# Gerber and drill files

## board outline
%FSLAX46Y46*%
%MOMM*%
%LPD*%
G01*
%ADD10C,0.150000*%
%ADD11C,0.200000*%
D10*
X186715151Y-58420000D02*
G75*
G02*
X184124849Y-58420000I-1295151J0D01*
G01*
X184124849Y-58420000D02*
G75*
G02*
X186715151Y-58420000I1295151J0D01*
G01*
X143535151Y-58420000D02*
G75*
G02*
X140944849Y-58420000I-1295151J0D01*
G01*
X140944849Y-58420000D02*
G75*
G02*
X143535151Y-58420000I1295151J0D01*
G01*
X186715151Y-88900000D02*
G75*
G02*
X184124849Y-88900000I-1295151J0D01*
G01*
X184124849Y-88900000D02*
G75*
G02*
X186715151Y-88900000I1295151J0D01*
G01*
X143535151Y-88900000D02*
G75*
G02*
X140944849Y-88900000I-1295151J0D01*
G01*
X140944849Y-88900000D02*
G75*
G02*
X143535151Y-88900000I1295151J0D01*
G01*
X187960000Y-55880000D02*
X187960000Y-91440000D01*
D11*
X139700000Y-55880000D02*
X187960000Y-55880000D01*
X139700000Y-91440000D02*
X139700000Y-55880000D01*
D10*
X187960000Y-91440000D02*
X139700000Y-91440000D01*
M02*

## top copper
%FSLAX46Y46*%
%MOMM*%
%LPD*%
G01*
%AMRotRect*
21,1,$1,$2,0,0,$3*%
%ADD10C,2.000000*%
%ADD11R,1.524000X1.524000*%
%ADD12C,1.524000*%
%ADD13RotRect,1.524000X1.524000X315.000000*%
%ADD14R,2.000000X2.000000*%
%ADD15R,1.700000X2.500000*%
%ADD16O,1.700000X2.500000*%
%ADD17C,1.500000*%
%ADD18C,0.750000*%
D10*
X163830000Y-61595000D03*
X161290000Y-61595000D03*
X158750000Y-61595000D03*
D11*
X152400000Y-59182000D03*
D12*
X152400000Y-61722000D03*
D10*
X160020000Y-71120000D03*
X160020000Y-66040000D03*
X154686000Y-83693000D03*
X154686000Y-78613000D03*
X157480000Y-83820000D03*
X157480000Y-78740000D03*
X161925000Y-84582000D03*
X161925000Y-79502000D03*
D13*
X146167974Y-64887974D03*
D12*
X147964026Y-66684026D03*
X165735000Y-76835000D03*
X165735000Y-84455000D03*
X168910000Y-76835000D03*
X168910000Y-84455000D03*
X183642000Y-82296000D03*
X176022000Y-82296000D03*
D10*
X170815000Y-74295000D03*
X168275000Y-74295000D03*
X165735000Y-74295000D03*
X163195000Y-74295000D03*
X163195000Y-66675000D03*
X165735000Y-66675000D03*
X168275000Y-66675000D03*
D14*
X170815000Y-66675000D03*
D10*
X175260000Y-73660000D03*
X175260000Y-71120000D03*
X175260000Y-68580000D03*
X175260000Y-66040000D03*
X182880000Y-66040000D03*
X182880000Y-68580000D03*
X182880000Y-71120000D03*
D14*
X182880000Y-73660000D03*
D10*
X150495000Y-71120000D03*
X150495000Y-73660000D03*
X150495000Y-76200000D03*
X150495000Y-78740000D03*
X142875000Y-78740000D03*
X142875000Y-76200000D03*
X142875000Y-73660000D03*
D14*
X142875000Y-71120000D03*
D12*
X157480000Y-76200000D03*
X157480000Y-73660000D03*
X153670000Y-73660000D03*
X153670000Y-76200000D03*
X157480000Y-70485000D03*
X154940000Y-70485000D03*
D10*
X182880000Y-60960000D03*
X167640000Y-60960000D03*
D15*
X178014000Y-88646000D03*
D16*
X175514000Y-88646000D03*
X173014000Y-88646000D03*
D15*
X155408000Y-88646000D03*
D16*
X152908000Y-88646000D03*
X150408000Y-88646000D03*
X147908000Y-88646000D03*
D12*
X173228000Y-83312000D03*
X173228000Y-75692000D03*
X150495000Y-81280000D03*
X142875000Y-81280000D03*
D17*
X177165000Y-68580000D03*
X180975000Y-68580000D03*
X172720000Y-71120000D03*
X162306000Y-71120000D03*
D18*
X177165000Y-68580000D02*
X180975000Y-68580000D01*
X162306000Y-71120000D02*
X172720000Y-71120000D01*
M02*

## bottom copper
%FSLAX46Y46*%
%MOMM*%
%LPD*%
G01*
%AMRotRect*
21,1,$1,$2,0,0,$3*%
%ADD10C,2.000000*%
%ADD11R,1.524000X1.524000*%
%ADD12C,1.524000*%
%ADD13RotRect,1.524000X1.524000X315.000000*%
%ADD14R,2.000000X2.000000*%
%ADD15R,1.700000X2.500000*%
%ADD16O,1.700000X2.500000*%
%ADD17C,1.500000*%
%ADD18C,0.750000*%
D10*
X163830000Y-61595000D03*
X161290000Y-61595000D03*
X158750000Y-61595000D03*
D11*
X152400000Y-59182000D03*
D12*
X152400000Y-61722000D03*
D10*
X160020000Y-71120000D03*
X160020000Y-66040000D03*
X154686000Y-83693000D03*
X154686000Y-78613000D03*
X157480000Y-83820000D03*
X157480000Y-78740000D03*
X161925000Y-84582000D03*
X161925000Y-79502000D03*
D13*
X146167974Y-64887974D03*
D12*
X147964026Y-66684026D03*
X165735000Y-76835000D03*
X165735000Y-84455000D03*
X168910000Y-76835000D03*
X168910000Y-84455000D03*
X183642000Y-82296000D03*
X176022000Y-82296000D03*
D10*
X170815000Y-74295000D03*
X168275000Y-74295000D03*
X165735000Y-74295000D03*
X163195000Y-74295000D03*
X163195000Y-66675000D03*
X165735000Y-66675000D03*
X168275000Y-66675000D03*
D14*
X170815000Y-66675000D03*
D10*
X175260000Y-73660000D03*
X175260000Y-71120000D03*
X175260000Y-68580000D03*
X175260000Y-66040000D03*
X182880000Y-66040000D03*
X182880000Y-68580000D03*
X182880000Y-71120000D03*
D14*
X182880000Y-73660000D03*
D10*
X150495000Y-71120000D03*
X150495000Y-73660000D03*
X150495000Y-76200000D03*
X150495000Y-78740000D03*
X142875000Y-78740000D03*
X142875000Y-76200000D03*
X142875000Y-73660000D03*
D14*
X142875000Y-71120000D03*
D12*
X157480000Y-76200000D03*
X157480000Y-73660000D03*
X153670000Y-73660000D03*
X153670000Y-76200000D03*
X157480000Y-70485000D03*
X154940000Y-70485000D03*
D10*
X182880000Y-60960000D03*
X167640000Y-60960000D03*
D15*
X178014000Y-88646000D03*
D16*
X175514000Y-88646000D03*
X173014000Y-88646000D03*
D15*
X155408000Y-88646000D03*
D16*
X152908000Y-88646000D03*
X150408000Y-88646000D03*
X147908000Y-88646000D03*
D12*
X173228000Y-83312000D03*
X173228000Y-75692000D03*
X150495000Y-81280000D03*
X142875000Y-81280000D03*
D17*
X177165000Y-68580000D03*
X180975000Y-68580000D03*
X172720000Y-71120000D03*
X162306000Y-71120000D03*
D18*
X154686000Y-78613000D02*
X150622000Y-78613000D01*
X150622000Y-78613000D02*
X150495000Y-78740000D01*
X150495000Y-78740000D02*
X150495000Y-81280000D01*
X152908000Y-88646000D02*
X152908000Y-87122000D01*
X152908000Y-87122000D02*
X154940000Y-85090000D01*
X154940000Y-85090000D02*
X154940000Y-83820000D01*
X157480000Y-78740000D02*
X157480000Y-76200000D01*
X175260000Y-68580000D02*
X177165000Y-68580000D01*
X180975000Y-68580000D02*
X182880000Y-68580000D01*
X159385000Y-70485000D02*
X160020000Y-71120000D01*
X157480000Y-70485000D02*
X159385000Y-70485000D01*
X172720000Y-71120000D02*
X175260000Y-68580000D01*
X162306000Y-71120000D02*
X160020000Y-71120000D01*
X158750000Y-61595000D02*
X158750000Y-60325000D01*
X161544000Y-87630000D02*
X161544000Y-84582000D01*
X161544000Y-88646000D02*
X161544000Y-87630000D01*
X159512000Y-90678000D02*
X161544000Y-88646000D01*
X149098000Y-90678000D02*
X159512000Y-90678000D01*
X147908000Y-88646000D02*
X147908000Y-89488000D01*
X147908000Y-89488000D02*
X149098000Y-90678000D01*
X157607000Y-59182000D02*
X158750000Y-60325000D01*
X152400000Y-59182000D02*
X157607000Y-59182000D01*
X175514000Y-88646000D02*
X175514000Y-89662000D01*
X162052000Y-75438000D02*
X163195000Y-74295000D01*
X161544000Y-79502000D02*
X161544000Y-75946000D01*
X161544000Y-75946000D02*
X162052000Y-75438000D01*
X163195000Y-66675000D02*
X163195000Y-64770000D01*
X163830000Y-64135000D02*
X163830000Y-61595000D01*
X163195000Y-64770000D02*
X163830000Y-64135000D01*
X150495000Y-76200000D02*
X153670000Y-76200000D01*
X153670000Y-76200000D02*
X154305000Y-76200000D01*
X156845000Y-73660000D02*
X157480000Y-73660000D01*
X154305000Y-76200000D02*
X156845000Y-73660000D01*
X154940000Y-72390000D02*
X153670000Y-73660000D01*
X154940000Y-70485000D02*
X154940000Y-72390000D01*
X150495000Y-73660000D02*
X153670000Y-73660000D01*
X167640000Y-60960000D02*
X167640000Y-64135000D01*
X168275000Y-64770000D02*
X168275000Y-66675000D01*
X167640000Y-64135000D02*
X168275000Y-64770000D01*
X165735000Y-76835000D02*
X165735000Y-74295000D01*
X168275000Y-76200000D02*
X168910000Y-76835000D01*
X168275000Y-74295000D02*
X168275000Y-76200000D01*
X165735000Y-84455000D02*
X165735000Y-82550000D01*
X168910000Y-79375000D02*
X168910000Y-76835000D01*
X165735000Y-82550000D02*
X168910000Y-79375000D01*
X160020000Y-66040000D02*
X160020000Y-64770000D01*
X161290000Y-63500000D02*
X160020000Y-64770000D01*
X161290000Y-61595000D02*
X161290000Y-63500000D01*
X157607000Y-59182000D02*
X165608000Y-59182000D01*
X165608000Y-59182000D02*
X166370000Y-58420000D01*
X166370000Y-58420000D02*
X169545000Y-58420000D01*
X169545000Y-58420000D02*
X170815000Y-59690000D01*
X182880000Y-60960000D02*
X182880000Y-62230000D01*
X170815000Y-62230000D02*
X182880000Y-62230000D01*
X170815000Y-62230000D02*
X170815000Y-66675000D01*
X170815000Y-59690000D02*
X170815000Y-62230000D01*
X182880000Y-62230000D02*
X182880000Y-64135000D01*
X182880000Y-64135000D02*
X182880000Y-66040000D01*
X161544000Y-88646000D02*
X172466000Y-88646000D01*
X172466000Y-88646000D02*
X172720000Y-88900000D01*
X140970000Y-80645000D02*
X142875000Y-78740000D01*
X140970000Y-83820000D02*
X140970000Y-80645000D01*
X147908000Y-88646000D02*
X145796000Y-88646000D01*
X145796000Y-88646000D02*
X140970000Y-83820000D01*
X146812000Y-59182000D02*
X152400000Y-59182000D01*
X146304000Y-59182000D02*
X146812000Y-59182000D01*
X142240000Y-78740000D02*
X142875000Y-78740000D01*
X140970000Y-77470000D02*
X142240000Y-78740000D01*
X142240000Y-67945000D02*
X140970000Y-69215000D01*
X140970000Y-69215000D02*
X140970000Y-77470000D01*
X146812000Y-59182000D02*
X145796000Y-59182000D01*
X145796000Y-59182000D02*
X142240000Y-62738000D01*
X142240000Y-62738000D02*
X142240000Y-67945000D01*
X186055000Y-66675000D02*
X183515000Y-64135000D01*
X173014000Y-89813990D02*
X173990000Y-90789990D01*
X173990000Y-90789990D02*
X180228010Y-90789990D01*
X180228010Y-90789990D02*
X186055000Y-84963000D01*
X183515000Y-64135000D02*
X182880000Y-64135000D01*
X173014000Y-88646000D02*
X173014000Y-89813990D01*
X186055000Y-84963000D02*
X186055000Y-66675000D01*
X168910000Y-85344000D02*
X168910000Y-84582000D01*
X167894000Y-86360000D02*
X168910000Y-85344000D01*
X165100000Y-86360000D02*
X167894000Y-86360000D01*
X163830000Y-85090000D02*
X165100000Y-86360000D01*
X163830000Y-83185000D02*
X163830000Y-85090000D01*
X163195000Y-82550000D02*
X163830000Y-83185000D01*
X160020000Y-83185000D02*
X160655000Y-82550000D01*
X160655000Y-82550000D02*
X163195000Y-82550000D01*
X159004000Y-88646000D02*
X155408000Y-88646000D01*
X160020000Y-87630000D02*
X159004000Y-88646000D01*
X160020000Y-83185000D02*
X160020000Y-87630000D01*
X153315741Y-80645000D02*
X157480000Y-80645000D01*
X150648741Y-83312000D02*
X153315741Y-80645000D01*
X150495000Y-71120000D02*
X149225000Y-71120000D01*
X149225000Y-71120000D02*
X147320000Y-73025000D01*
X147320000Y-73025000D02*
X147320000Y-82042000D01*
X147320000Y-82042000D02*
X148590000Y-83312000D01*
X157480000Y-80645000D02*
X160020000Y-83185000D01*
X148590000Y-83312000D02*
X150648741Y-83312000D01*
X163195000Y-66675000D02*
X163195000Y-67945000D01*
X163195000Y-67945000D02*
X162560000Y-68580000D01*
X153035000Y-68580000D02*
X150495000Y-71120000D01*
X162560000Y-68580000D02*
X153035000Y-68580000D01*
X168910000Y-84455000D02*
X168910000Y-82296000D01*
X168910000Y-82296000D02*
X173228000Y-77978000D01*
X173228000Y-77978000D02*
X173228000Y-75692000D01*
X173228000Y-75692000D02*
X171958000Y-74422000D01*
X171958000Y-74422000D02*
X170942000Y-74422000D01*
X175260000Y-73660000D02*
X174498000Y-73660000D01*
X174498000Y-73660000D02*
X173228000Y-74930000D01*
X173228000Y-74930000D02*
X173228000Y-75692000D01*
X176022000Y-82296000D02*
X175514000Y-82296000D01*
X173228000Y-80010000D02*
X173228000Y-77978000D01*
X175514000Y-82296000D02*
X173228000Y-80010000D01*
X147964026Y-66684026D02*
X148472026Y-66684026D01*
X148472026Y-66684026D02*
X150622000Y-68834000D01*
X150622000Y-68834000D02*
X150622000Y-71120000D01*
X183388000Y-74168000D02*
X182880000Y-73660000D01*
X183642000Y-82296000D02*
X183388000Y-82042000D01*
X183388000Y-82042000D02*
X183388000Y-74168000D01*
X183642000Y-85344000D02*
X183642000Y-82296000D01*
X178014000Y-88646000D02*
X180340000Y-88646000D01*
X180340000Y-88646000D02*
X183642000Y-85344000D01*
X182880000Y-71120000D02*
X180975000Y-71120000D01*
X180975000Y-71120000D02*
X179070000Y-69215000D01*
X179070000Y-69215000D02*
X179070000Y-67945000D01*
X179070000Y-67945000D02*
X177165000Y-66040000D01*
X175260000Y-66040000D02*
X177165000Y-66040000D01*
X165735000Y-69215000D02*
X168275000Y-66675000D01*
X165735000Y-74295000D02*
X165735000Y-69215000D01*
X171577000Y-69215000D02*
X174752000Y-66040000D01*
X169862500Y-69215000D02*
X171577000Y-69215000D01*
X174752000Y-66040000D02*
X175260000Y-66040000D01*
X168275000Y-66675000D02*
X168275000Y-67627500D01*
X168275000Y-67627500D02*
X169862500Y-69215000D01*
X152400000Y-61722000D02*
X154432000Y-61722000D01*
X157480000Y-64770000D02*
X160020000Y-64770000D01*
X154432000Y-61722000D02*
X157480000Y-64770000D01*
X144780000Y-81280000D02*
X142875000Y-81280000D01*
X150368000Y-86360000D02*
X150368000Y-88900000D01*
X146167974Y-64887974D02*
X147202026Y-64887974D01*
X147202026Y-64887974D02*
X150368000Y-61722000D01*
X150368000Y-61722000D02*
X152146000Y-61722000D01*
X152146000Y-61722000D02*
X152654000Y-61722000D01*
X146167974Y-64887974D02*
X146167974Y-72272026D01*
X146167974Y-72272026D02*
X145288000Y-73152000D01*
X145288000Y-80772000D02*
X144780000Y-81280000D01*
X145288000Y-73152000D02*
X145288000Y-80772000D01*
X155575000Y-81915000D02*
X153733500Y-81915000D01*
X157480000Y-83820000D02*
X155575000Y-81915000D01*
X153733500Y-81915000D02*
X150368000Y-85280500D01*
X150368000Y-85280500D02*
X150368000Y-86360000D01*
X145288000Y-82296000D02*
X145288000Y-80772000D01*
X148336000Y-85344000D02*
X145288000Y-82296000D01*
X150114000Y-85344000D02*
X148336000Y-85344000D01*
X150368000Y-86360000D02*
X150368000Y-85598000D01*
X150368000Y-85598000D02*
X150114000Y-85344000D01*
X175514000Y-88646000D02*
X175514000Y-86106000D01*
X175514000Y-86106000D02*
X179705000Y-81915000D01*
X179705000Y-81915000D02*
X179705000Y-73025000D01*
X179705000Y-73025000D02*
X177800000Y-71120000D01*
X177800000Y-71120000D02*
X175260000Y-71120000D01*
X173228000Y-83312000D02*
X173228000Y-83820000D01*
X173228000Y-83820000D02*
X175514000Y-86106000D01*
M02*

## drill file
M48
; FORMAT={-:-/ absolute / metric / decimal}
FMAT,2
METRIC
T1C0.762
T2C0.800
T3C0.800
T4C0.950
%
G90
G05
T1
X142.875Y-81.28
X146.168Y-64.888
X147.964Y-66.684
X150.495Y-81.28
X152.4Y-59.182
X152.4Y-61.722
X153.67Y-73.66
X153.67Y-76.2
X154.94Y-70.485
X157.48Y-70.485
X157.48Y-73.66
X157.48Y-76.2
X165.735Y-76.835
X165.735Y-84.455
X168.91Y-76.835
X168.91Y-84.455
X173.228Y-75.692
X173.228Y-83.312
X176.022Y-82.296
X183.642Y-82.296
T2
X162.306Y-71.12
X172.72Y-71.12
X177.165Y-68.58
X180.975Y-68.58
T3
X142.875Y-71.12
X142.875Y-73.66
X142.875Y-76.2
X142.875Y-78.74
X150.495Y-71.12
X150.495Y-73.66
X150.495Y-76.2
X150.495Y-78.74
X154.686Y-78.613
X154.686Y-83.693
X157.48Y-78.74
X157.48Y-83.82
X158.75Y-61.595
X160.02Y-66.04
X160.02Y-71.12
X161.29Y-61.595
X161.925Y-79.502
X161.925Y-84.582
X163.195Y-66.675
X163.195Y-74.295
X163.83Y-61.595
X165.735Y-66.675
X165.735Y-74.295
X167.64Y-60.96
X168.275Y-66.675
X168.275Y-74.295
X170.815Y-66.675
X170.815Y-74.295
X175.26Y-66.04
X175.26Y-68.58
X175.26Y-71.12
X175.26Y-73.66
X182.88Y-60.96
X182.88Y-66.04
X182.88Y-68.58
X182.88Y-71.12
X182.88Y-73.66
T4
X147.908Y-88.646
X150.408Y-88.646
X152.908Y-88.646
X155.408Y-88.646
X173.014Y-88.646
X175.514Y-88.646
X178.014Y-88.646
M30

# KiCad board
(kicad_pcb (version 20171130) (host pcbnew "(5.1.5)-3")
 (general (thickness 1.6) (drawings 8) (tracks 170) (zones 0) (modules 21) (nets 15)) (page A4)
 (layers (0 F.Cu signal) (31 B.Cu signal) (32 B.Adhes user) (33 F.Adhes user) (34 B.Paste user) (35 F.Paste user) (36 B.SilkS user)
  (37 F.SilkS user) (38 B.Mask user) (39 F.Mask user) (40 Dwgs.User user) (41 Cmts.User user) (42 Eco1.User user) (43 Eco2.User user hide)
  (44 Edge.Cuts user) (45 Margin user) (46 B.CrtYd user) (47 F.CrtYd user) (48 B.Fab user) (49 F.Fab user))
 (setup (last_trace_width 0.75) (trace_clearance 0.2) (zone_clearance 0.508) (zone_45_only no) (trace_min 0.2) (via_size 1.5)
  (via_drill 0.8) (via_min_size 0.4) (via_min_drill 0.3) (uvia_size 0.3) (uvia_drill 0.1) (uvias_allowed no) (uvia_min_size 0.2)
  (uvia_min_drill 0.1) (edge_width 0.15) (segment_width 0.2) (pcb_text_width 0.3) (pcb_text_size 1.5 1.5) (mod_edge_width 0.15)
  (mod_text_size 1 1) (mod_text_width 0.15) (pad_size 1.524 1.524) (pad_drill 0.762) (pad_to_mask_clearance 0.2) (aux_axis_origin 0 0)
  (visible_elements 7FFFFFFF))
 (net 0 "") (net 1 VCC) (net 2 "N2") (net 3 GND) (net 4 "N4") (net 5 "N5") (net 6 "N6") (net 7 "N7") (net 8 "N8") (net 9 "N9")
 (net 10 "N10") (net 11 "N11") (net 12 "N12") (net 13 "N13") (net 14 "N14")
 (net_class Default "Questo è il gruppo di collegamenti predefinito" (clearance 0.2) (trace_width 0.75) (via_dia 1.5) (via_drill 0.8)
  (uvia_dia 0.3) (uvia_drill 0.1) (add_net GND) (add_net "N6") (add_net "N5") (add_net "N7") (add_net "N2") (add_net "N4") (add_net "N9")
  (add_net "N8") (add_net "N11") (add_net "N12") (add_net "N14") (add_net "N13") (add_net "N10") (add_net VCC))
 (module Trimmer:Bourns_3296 (layer F.Cu) (at 158.75 61.595 180)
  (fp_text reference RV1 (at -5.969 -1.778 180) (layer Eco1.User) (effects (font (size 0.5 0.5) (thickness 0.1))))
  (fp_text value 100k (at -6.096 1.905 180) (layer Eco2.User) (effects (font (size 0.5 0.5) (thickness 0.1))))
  (pad 3 thru_hole circle (at -5.08 0 180) (size 2 2) (drill 0.8) (layers *.Cu *.Mask) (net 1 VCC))
  (pad 2 thru_hole circle (at -2.54 0 180) (size 2 2) (drill 0.8) (layers *.Cu *.Mask) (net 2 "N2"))
  (pad 1 thru_hole circle (at 0 0 180) (size 2 2) (drill 0.8) (layers *.Cu *.Mask) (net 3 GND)))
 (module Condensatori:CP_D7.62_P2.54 (layer F.Cu) (at 152.4 60.452 270)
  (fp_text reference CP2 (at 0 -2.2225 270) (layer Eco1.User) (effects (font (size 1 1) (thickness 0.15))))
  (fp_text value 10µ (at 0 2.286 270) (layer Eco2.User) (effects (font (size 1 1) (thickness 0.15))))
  (pad 1 thru_hole rect (at -1.27 0 270) (size 1.524 1.524) (drill 0.762) (layers *.Cu *.Mask) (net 3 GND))
  (pad 2 thru_hole circle (at 1.27 0 270) (size 1.524 1.524) (drill 0.762) (layers *.Cu *.Mask) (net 2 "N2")))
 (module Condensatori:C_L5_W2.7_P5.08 (layer F.Cu) (at 160.02 66.04 270)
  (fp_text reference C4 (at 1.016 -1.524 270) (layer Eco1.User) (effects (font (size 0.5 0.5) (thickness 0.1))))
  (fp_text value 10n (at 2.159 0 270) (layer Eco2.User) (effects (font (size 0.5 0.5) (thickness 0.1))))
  (pad 2 thru_hole circle (at 5.08 0 270) (size 2 2) (drill 0.8) (layers *.Cu *.Mask) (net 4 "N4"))
  (pad 1 thru_hole circle (at 0 0 270) (size 2 2) (drill 0.8) (layers *.Cu *.Mask) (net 2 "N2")))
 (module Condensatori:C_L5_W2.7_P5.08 (layer F.Cu) (at 154.686 78.613 270)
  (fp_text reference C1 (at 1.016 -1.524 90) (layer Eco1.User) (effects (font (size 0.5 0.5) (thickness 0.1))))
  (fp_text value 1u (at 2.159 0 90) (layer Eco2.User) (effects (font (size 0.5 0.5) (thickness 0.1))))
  (pad 2 thru_hole circle (at 5.08 0 270) (size 2 2) (drill 0.8) (layers *.Cu *.Mask) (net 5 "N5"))
  (pad 1 thru_hole circle (at 0 0 270) (size 2 2) (drill 0.8) (layers *.Cu *.Mask) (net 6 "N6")))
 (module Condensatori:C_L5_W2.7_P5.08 (layer F.Cu) (at 157.48 78.74 270)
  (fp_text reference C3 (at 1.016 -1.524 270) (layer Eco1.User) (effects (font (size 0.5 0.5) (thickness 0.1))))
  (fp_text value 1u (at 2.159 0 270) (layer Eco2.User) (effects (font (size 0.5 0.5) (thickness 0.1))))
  (pad 2 thru_hole circle (at 5.08 0 270) (size 2 2) (drill 0.8) (layers *.Cu *.Mask) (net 2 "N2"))
  (pad 1 thru_hole circle (at 0 0 270) (size 2 2) (drill 0.8) (layers *.Cu *.Mask) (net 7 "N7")))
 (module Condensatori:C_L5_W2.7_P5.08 (layer F.Cu) (at 161.925 79.502 270)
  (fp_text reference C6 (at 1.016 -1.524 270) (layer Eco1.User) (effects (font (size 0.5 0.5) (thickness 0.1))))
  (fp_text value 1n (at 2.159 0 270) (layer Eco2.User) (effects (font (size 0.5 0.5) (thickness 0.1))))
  (pad 2 thru_hole circle (at 5.08 0 270) (size 2 2) (drill 0.8) (layers *.Cu *.Mask) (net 3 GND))
  (pad 1 thru_hole circle (at 0 0 270) (size 2 2) (drill 0.8) (layers *.Cu *.Mask) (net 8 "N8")))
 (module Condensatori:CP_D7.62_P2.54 (layer F.Cu) (at 147.066 65.786 315)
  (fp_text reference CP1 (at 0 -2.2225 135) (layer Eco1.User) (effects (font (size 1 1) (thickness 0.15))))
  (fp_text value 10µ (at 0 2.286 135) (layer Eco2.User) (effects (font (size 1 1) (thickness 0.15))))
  (pad 1 thru_hole rect (at -1.27 0 315) (size 1.524 1.524) (drill 0.762) (layers *.Cu *.Mask) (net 2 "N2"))
  (pad 2 thru_hole circle (at 1.27 0 315) (size 1.524 1.524) (drill 0.762) (layers *.Cu *.Mask) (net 1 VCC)))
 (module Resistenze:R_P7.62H (layer F.Cu) (at 165.735 80.645 90)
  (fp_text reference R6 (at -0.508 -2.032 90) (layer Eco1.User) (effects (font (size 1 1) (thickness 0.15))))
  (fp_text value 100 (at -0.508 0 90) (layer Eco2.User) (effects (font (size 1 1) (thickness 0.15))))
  (pad 2 thru_hole circle (at 3.81 0 90) (size 1.524 1.524) (drill 0.762) (layers *.Cu *.Mask) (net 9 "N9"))
  (pad 1 thru_hole circle (at -3.81 0 90) (size 1.524 1.524) (drill 0.762) (layers *.Cu *.Mask) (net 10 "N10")))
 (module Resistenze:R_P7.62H (layer F.Cu) (at 168.91 80.645 90)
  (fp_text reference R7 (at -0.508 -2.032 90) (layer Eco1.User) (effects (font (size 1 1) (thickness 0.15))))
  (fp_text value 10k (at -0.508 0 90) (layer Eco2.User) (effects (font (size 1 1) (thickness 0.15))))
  (pad 2 thru_hole circle (at 3.81 0 90) (size 1.524 1.524) (drill 0.762) (layers *.Cu *.Mask) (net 10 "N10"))
  (pad 1 thru_hole circle (at -3.81 0 90) (size 1.524 1.524) (drill 0.762) (layers *.Cu *.Mask) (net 1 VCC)))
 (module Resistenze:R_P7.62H (layer F.Cu) (at 179.832 82.296)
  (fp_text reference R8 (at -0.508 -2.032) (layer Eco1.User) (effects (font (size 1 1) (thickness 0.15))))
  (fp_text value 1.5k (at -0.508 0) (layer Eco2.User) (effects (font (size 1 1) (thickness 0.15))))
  (pad 2 thru_hole circle (at 3.81 0) (size 1.524 1.524) (drill 0.762) (layers *.Cu *.Mask) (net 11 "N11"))
  (pad 1 thru_hole circle (at -3.81 0) (size 1.524 1.524) (drill 0.762) (layers *.Cu *.Mask) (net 1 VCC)))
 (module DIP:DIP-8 (layer F.Cu) (at 170.815 66.675 270)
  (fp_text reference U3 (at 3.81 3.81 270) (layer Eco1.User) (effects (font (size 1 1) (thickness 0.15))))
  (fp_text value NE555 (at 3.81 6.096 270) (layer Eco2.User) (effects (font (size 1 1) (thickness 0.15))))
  (pad 8 thru_hole circle (at 7.62 0 180) (size 2 2) (drill 0.8) (layers *.Cu *.Mask) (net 1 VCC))
  (pad 7 thru_hole circle (at 7.62 2.54 180) (size 2 2) (drill 0.8) (layers *.Cu *.Mask) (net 10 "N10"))
  (pad 6 thru_hole circle (at 7.62 5.08 180) (size 2 2) (drill 0.8) (layers *.Cu *.Mask) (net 9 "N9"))
  (pad 5 thru_hole circle (at 7.62 7.62 180) (size 2 2) (drill 0.8) (layers *.Cu *.Mask) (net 8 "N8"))
  (pad 4 thru_hole circle (at 0 7.62 180) (size 2 2) (drill 0.8) (layers *.Cu *.Mask) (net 1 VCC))
  (pad 3 thru_hole circle (at 0 5.08 180) (size 2 2) (drill 0.8) (layers *.Cu *.Mask))
  (pad 2 thru_hole circle (at 0 2.54 180) (size 2 2) (drill 0.8) (layers *.Cu *.Mask) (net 9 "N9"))
  (pad 1 thru_hole rect (at 0 0 180) (size 2 2) (drill 0.8) (layers *.Cu *.Mask) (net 3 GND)))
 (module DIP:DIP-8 (layer F.Cu) (at 182.88 73.66 180)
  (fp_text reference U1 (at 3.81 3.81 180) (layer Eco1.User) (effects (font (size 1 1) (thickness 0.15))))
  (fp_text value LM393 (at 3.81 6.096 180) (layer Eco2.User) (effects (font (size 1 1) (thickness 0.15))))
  (pad 8 thru_hole circle (at 7.62 0 90) (size 2 2) (drill 0.8) (layers *.Cu *.Mask) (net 1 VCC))
  (pad 7 thru_hole circle (at 7.62 2.54 90) (size 2 2) (drill 0.8) (layers *.Cu *.Mask) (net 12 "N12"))
  (pad 6 thru_hole circle (at 7.62 5.08 90) (size 2 2) (drill 0.8) (layers *.Cu *.Mask) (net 4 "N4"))
  (pad 5 thru_hole circle (at 7.62 7.62 90) (size 2 2) (drill 0.8) (layers *.Cu *.Mask) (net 9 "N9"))
  (pad 4 thru_hole circle (at 0 7.62 90) (size 2 2) (drill 0.8) (layers *.Cu *.Mask) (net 3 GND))
  (pad 3 thru_hole circle (at 0 5.08 90) (size 2 2) (drill 0.8) (layers *.Cu *.Mask) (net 4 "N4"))
  (pad 2 thru_hole circle (at 0 2.54 90) (size 2 2) (drill 0.8) (layers *.Cu *.Mask) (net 9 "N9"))
  (pad 1 thru_hole rect (at 0 0 90) (size 2 2) (drill 0.8) (layers *.Cu *.Mask) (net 11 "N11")))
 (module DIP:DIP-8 (layer F.Cu) (at 142.875 71.12)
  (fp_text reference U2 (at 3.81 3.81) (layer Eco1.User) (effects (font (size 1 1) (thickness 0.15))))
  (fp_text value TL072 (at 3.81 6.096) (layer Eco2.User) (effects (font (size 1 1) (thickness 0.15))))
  (pad 8 thru_hole circle (at 7.62 0 270) (size 2 2) (drill 0.8) (layers *.Cu *.Mask) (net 1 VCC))
  (pad 7 thru_hole circle (at 7.62 2.54 270) (size 2 2) (drill 0.8) (layers *.Cu *.Mask) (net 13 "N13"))
  (pad 6 thru_hole circle (at 7.62 5.08 270) (size 2 2) (drill 0.8) (layers *.Cu *.Mask) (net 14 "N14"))
  (pad 5 thru_hole circle (at 7.62 7.62 270) (size 2 2) (drill 0.8) (layers *.Cu *.Mask) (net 6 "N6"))
  (pad 4 thru_hole circle (at 0 7.62 270) (size 2 2) (drill 0.8) (layers *.Cu *.Mask) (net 3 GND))
  (pad 3 thru_hole circle (at 0 5.08 270) (size 2 2) (drill 0.8) (layers *.Cu *.Mask))
  (pad 2 thru_hole circle (at 0 2.54 270) (size 2 2) (drill 0.8) (layers *.Cu *.Mask))
  (pad 1 thru_hole rect (at 0 0 270) (size 2 2) (drill 0.8) (layers *.Cu *.Mask)))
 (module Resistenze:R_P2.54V (layer F.Cu) (at 157.48 73.66 270)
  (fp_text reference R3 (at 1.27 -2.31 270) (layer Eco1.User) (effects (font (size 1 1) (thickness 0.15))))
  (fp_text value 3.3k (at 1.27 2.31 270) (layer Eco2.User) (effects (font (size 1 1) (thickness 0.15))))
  (pad 2 thru_hole circle (at 2.54 0 270) (size 1.524 1.524) (drill 0.762) (layers *.Cu *.Mask) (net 7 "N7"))
  (pad 1 thru_hole circle (at 0 0 270) (size 1.524 1.524) (drill 0.762) (layers *.Cu *.Mask) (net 14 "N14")))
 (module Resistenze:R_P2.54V (layer F.Cu) (at 153.67 76.2 90)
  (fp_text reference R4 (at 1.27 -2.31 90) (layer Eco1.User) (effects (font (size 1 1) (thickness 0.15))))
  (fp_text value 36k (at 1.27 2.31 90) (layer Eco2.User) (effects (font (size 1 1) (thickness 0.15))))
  (pad 2 thru_hole circle (at 2.54 0 90) (size 1.524 1.524) (drill 0.762) (layers *.Cu *.Mask) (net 13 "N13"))
  (pad 1 thru_hole circle (at 0 0 90) (size 1.524 1.524) (drill 0.762) (layers *.Cu *.Mask) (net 14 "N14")))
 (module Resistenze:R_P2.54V (layer F.Cu) (at 154.94 70.485)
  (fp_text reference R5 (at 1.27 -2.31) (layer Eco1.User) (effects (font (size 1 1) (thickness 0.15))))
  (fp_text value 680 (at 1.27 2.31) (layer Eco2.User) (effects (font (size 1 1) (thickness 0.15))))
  (pad 2 thru_hole circle (at 2.54 0) (size 1.524 1.524) (drill 0.762) (layers *.Cu *.Mask) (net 4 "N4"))
  (pad 1 thru_hole circle (at 0 0) (size 1.524 1.524) (drill 0.762) (layers *.Cu *.Mask) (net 13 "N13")))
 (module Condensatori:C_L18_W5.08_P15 (layer F.Cu) (at 167.64 60.96)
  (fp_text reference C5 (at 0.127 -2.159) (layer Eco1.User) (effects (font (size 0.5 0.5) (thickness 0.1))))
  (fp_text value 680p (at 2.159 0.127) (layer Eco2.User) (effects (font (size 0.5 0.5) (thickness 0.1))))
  (pad 2 thru_hole circle (at 15.24 0) (size 2 2) (drill 0.8) (layers *.Cu *.Mask) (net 3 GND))
  (pad 1 thru_hole circle (at 0 0) (size 2 2) (drill 0.8) (layers *.Cu *.Mask) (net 9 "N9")))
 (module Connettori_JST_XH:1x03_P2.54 (layer F.Cu) (at 178.014 88.646 180)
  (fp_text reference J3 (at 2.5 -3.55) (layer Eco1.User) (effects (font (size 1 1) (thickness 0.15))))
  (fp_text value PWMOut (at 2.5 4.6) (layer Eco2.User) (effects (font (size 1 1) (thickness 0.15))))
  (pad 1 thru_hole rect (at 0 0 180) (size 1.7 2.5) (drill 0.95) (layers *.Cu *.Mask) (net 11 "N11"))
  (pad 2 thru_hole oval (at 2.5 0 180) (size 1.7 2.5) (drill 0.95) (layers *.Cu *.Mask) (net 12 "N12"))
  (pad 3 thru_hole oval (at 5 0 180) (size 1.7 2.5) (drill 0.95) (layers *.Cu *.Mask) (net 3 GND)))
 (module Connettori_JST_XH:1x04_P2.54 (layer F.Cu) (at 155.408 88.646 180)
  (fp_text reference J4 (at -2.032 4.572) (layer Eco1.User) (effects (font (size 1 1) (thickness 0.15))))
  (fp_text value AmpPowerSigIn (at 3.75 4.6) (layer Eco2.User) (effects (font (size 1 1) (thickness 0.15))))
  (pad 1 thru_hole rect (at 0 0 180) (size 1.7 2.5) (drill 0.95) (layers *.Cu *.Mask) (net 1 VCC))
  (pad 2 thru_hole oval (at 2.5 0 180) (size 1.7 2.5) (drill 0.95) (layers *.Cu *.Mask) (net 5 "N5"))
  (pad 3 thru_hole oval (at 5 0 180) (size 1.7 2.5) (drill 0.95) (layers *.Cu *.Mask) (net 2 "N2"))
  (pad 4 thru_hole oval (at 7.5 0 180) (size 1.7 2.5) (drill 0.95) (layers *.Cu *.Mask) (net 3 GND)))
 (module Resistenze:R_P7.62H (layer F.Cu) (at 173.228 79.502 270)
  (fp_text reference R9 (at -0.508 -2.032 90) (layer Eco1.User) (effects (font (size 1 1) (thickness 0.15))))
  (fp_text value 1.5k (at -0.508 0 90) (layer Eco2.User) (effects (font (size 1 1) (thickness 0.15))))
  (pad 2 thru_hole circle (at 3.81 0 270) (size 1.524 1.524) (drill 0.762) (layers *.Cu *.Mask) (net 12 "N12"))
  (pad 1 thru_hole circle (at -3.81 0 270) (size 1.524 1.524) (drill 0.762) (layers *.Cu *.Mask) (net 1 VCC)))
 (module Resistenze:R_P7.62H (layer F.Cu) (at 146.685 81.28)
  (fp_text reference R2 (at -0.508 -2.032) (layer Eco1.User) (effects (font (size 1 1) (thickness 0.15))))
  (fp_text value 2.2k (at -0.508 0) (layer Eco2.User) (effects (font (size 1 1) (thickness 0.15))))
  (pad 2 thru_hole circle (at 3.81 0) (size 1.524 1.524) (drill 0.762) (layers *.Cu *.Mask) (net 6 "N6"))
  (pad 1 thru_hole circle (at -3.81 0) (size 1.524 1.524) (drill 0.762) (layers *.Cu *.Mask) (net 2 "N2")))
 (gr_circle (center 185.42 58.42) (end 186.69 58.674) (layer Edge.Cuts) (width 0.15))
 (gr_circle (center 142.24 58.42) (end 143.51 58.674) (layer Edge.Cuts) (width 0.15))
 (gr_circle (center 185.42 88.9) (end 186.69 89.154) (layer Edge.Cuts) (width 0.15))
 (gr_circle (center 142.24 88.9) (end 143.51 89.154) (layer Edge.Cuts) (width 0.15))
 (gr_line (start 187.96 55.88) (end 187.96 91.44) (layer Edge.Cuts) (width 0.15))
 (gr_line (start 139.7 55.88) (end 187.96 55.88) (layer Edge.Cuts) (width 0.2))
 (gr_line (start 139.7 91.44) (end 139.7 55.88) (layer Edge.Cuts) (width 0.2))
 (gr_line (start 187.96 91.44) (end 139.7 91.44) (layer Edge.Cuts) (width 0.15))
 (segment (start 154.686 78.613) (end 150.622 78.613) (width 0.75) (layer B.Cu) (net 6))
 (segment (start 150.622 78.613) (end 150.495 78.74) (width 0.75) (layer B.Cu) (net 6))
 (segment (start 150.495 78.74) (end 150.495 81.28) (width 0.75) (layer B.Cu) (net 6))
 (segment (start 152.908 88.646) (end 152.908 87.122) (width 0.75) (layer B.Cu) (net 5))
 (segment (start 152.908 87.122) (end 154.94 85.09) (width 0.75) (layer B.Cu) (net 5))
 (segment (start 154.94 85.09) (end 154.94 83.82) (width 0.75) (layer B.Cu) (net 5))
 (segment (start 157.48 78.74) (end 157.48 76.2) (width 0.75) (layer B.Cu) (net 7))
 (via (at 177.165 68.58) (size 1.5) (drill 0.8) (layers F.Cu B.Cu) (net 4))
 (segment (start 175.26 68.58) (end 177.165 68.58) (width 0.75) (layer B.Cu) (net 4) (status 10))
 (via (at 180.975 68.58) (size 1.5) (drill 0.8) (layers F.Cu B.Cu) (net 4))
 (segment (start 180.975 68.58) (end 182.88 68.58) (width 0.75) (layer B.Cu) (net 4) (status 20))
 (segment (start 177.165 68.58) (end 180.975 68.58) (width 0.75) (layer F.Cu) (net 4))
 (segment (start 159.385 70.485) (end 160.02 71.12) (width 0.75) (layer B.Cu) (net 4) (status 30))
 (segment (start 157.48 70.485) (end 159.385 70.485) (width 0.75) (layer B.Cu) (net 4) (status 30))
 (via (at 172.72 71.12) (size 1.5) (drill 0.8) (layers F.Cu B.Cu) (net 4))
 (segment (start 172.72 71.12) (end 175.26 68.58) (width 0.75) (layer B.Cu) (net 4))
 (via (at 162.306 71.12) (size 1.5) (drill 0.8) (layers F.Cu B.Cu) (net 4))
 (segment (start 162.306 71.12) (end 160.02 71.12) (width 0.75) (layer B.Cu) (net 4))
 (segment (start 162.306 71.12) (end 172.72 71.12) (width 0.75) (layer F.Cu) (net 4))
 (segment (start 158.75 61.595) (end 158.75 60.325) (width 0.75) (layer B.Cu) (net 3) (status 10))
 (segment (start 161.544 87.63) (end 161.544 84.582) (width 0.75) (layer B.Cu) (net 3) (status 20))
 (segment (start 161.544 88.646) (end 161.544 87.63) (width 0.75) (layer B.Cu) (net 3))
 (segment (start 159.512 90.678) (end 161.544 88.646) (width 0.75) (layer B.Cu) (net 3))
 (segment (start 149.098 90.678) (end 159.512 90.678) (width 0.75) (layer B.Cu) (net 3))
 (segment (start 147.908 88.646) (end 147.908 89.488) (width 0.75) (layer B.Cu) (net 3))
 (segment (start 147.908 89.488) (end 149.098 90.678) (width 0.75) (layer B.Cu) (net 3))
 (segment (start 157.607 59.182) (end 158.75 60.325) (width 0.75) (layer B.Cu) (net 3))
 (segment (start 152.4 59.182) (end 157.607 59.182) (width 0.75) (layer B.Cu) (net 3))
 (segment (start 175.514 88.646) (end 175.514 89.662) (width 0.75) (layer B.Cu) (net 12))
 (segment (start 162.052 75.438) (end 163.195 74.295) (width 0.75) (layer B.Cu) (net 8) (status 20))
 (segment (start 161.544 79.502) (end 161.544 75.946) (width 0.75) (layer B.Cu) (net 8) (status 10))
 (segment (start 161.544 75.946) (end 162.052 75.438) (width 0.75) (layer B.Cu) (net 8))
 (segment (start 163.195 66.675) (end 163.195 64.77) (width 0.75) (layer B.Cu) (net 1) (status 10))
 (segment (start 163.83 64.135) (end 163.83 61.595) (width 0.75) (layer B.Cu) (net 1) (status 20))
 (segment (start 163.195 64.77) (end 163.83 64.135) (width 0.75) (layer B.Cu) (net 1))
 (segment (start 150.495 76.2) (end 153.67 76.2) (width 0.75) (layer B.Cu) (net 14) (status 30))
 (segment (start 153.67 76.2) (end 154.305 76.2) (width 0.75) (layer B.Cu) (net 14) (status 30))
 (segment (start 156.845 73.66) (end 157.48 73.66) (width 0.75) (layer B.Cu) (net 14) (status 30))
 (segment (start 154.305 76.2) (end 156.845 73.66) (width 0.75) (layer B.Cu) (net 14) (status 30))
 (segment (start 154.94 72.39) (end 153.67 73.66) (width 0.75) (layer B.Cu) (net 13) (status 20))
 (segment (start 154.94 70.485) (end 154.94 72.39) (width 0.75) (layer B.Cu) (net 13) (status 10))
 (segment (start 150.495 73.66) (end 153.67 73.66) (width 0.75) (layer B.Cu) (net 13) (status 30))
 (segment (start 167.64 60.96) (end 167.64 64.135) (width 0.75) (layer B.Cu) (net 9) (status 10))
 (segment (start 168.275 64.77) (end 168.275 66.675) (width 0.75) (layer B.Cu) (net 9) (status 20))
 (segment (start 167.64 64.135) (end 168.275 64.77) (width 0.75) (layer B.Cu) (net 9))
 (segment (start 165.735 76.835) (end 165.735 74.295) (width 0.75) (layer B.Cu) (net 9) (status 30))
 (segment (start 168.275 76.2) (end 168.91 76.835) (width 0.75) (layer B.Cu) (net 10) (status 20))
 (segment (start 168.275 74.295) (end 168.275 76.2) (width 0.75) (layer B.Cu) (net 10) (status 10))
 (segment (start 165.735 84.455) (end 165.735 82.55) (width 0.75) (layer B.Cu) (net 10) (status 10))
 (segment (start 168.91 79.375) (end 168.91 76.835) (width 0.75) (layer B.Cu) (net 10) (status 20))
 (segment (start 165.735 82.55) (end 168.91 79.375) (width 0.75) (layer B.Cu) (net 10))
 (segment (start 160.02 66.04) (end 160.02 64.77) (width 0.75) (layer B.Cu) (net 2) (status 10))
 (segment (start 161.29 63.5) (end 160.02 64.77) (width 0.75) (layer B.Cu) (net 2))
 (segment (start 161.29 61.595) (end 161.29 63.5) (width 0.75) (layer B.Cu) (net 2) (status 10))
 (segment (start 157.607 59.182) (end 165.608 59.182) (width 0.75) (layer B.Cu) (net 3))
 (segment (start 165.608 59.182) (end 166.37 58.42) (width 0.75) (layer B.Cu) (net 3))
 (segment (start 166.37 58.42) (end 169.545 58.42) (width 0.75) (layer B.Cu) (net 3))
 (segment (start 169.545 58.42) (end 170.815 59.69) (width 0.75) (layer B.Cu) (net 3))
 (segment (start 182.88 60.96) (end 182.88 62.23) (width 0.75) (layer B.Cu) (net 3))
 (segment (start 170.815 62.23) (end 182.88 62.23) (width 0.75) (layer B.Cu) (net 3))
 (segment (start 170.815 62.23) (end 170.815 66.675) (width 0.75) (layer B.Cu) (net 3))
 (segment (start 170.815 59.69) (end 170.815 62.23) (width 0.75) (layer B.Cu) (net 3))
 (segment (start 182.88 62.23) (end 182.88 64.135) (width 0.75) (layer B.Cu) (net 3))
 (segment (start 182.88 64.135) (end 182.88 66.04) (width 0.75) (layer B.Cu) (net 3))
 (segment (start 161.544 88.646) (end 172.466 88.646) (width 0.75) (layer B.Cu) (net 3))
 (segment (start 172.466 88.646) (end 172.72 88.9) (width 0.75) (layer B.Cu) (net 3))
 (segment (start 140.97 80.645) (end 142.875 78.74) (width 0.75) (layer B.Cu) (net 3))
 (segment (start 140.97 83.82) (end 140.97 80.645) (width 0.75) (layer B.Cu) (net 3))
 (segment (start 147.908 88.646) (end 145.796 88.646) (width 0.75) (layer B.Cu) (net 3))
 (segment (start 145.796 88.646) (end 140.97 83.82) (width 0.75) (layer B.Cu) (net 3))
 (segment (start 146.812 59.182) (end 152.4 59.182) (width 0.75) (layer B.Cu) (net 3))
 (segment (start 146.304 59.182) (end 146.812 59.182) (width 0.75) (layer B.Cu) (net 3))
 (segment (start 142.24 78.74) (end 142.875 78.74) (width 0.75) (layer B.Cu) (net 3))
 (segment (start 140.97 77.47) (end 142.24 78.74) (width 0.75) (layer B.Cu) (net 3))
 (segment (start 142.24 67.945) (end 140.97 69.215) (width 0.75) (layer B.Cu) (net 3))
 (segment (start 140.97 69.215) (end 140.97 77.47) (width 0.75) (layer B.Cu) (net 3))
 (segment (start 146.812 59.182) (end 145.796 59.182) (width 0.75) (layer B.Cu) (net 3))
 (segment (start 145.796 59.182) (end 142.24 62.738) (width 0.75) (layer B.Cu) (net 3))
 (segment (start 142.24 62.738) (end 142.24 67.945) (width 0.75) (layer B.Cu) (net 3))
 (segment (start 186.055 66.675) (end 183.515 64.135) (width 0.75) (layer B.Cu) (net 3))
 (segment (start 173.014 89.81399) (end 173.99 90.78999) (width 0.75) (layer B.Cu) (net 3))
 (segment (start 173.99 90.78999) (end 180.22801 90.78999) (width 0.75) (layer B.Cu) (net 3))
 (segment (start 180.22801 90.78999) (end 186.055 84.963) (width 0.75) (layer B.Cu) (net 3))
 (segment (start 183.515 64.135) (end 182.88 64.135) (width 0.75) (layer B.Cu) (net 3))
 (segment (start 173.014 88.646) (end 173.014 89.81399) (width 0.75) (layer B.Cu) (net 3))
 (segment (start 186.055 84.963) (end 186.055 66.675) (width 0.75) (layer B.Cu) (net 3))
 (segment (start 168.91 85.344) (end 168.91 84.582) (width 0.75) (layer B.Cu) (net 1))
 (segment (start 167.894 86.36) (end 168.91 85.344) (width 0.75) (layer B.Cu) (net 1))
 (segment (start 165.1 86.36) (end 167.894 86.36) (width 0.75) (layer B.Cu) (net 1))
 (segment (start 163.83 85.09) (end 165.1 86.36) (width 0.75) (layer B.Cu) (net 1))
 (segment (start 163.83 83.185) (end 163.83 85.09) (width 0.75) (layer B.Cu) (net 1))
 (segment (start 163.195 82.55) (end 163.83 83.185) (width 0.75) (layer B.Cu) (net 1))
 (segment (start 160.02 83.185) (end 160.655 82.55) (width 0.75) (layer B.Cu) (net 1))
 (segment (start 160.655 82.55) (end 163.195 82.55) (width 0.75) (layer B.Cu) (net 1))
 (segment (start 159.004 88.646) (end 155.408 88.646) (width 0.75) (layer B.Cu) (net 1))
 (segment (start 160.02 87.63) (end 159.004 88.646) (width 0.75) (layer B.Cu) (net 1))
 (segment (start 160.02 83.185) (end 160.02 87.63) (width 0.75) (layer B.Cu) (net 1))
 (segment (start 153.315741 80.645) (end 157.48 80.645) (width 0.75) (layer B.Cu) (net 1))
 (segment (start 150.648741 83.312) (end 153.315741 80.645) (width 0.75) (layer B.Cu) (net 1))
 (segment (start 150.495 71.12) (end 149.225 71.12) (width 0.75) (layer B.Cu) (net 1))
 (segment (start 149.225 71.12) (end 147.32 73.025) (width 0.75) (layer B.Cu) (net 1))
 (segment (start 147.32 73.025) (end 147.32 82.042) (width 0.75) (layer B.Cu) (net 1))
 (segment (start 147.32 82.042) (end 148.59 83.312) (width 0.75) (layer B.Cu) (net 1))
 (segment (start 157.48 80.645) (end 160.02 83.185) (width 0.75) (layer B.Cu) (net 1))
 (segment (start 148.59 83.312) (end 150.648741 83.312) (width 0.75) (layer B.Cu) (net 1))
 (segment (start 163.195 66.675) (end 163.195 67.945) (width 0.75) (layer B.Cu) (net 1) (status 10))
 (segment (start 163.195 67.945) (end 162.56 68.58) (width 0.75) (layer B.Cu) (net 1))
 (segment (start 153.035 68.58) (end 150.495 71.12) (width 0.75) (layer B.Cu) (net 1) (status 20))
 (segment (start 162.56 68.58) (end 153.035 68.58) (width 0.75) (layer B.Cu) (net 1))
 (segment (start 168.91 84.455) (end 168.91 82.296) (width 0.75) (layer B.Cu) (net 1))
 (segment (start 168.91 82.296) (end 173.228 77.978) (width 0.75) (layer B.Cu) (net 1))
 (segment (start 173.228 77.978) (end 173.228 75.692) (width 0.75) (layer B.Cu) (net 1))
 (segment (start 173.228 75.692) (end 171.958 74.422) (width 0.75) (layer B.Cu) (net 1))
 (segment (start 171.958 74.422) (end 170.942 74.422) (width 0.75) (layer B.Cu) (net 1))
 (segment (start 175.26 73.66) (end 174.498 73.66) (width 0.75) (layer B.Cu) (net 1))
 (segment (start 174.498 73.66) (end 173.228 74.93) (width 0.75) (layer B.Cu) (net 1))
 (segment (start 173.228 74.93) (end 173.228 75.692) (width 0.75) (layer B.Cu) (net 1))
 (segment (start 176.022 82.296) (end 175.514 82.296) (width 0.75) (layer B.Cu) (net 1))
 (segment (start 173.228 80.01) (end 173.228 77.978) (width 0.75) (layer B.Cu) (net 1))
 (segment (start 175.514 82.296) (end 173.228 80.01) (width 0.75) (layer B.Cu) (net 1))
 (segment (start 147.964026 66.684026) (end 148.472026 66.684026) (width 0.75) (layer B.Cu) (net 1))
 (segment (start 148.472026 66.684026) (end 150.622 68.834) (width 0.75) (layer B.Cu) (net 1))
 (segment (start 150.622 68.834) (end 150.622 71.12) (width 0.75) (layer B.Cu) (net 1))
 (segment (start 183.388 74.168) (end 182.88 73.66) (width 0.75) (layer B.Cu) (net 11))
 (segment (start 183.642 82.296) (end 183.388 82.042) (width 0.75) (layer B.Cu) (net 11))
 (segment (start 183.388 82.042) (end 183.388 74.168) (width 0.75) (layer B.Cu) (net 11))
 (segment (start 183.642 85.344) (end 183.642 82.296) (width 0.75) (layer B.Cu) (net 11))
 (segment (start 178.014 88.646) (end 180.34 88.646) (width 0.75) (layer B.Cu) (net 11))
 (segment (start 180.34 88.646) (end 183.642 85.344) (width 0.75) (layer B.Cu) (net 11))
 (segment (start 182.88 71.12) (end 180.975 71.12) (width 0.75) (layer B.Cu) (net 9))
 (segment (start 180.975 71.12) (end 179.07 69.215) (width 0.75) (layer B.Cu) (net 9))
 (segment (start 179.07 69.215) (end 179.07 67.945) (width 0.75) (layer B.Cu) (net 9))
 (segment (start 179.07 67.945) (end 177.165 66.04) (width 0.75) (layer B.Cu) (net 9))
 (segment (start 175.26 66.04) (end 177.165 66.04) (width 0.75) (layer B.Cu) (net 9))
 (segment (start 165.735 69.215) (end 168.275 66.675) (width 0.75) (layer B.Cu) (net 9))
 (segment (start 165.735 74.295) (end 165.735 69.215) (width 0.75) (layer B.Cu) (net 9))
 (segment (start 171.577 69.215) (end 174.752 66.04) (width 0.75) (layer B.Cu) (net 9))
 (segment (start 169.8625 69.215) (end 171.577 69.215) (width 0.75) (layer B.Cu) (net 9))
 (segment (start 174.752 66.04) (end 175.26 66.04) (width 0.75) (layer B.Cu) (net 9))
 (segment (start 168.275 66.675) (end 168.275 67.6275) (width 0.75) (layer B.Cu) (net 9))
 (segment (start 168.275 67.6275) (end 169.8625 69.215) (width 0.75) (layer B.Cu) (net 9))
 (segment (start 152.4 61.722) (end 154.432 61.722) (width 0.75) (layer B.Cu) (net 2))
 (segment (start 157.48 64.77) (end 160.02 64.77) (width 0.75) (layer B.Cu) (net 2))
 (segment (start 154.432 61.722) (end 157.48 64.77) (width 0.75) (layer B.Cu) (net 2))
 (segment (start 144.78 81.28) (end 142.875 81.28) (width 0.75) (layer B.Cu) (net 2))
 (segment (start 150.368 86.36) (end 150.368 88.9) (width 0.75) (layer B.Cu) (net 2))
 (segment (start 146.167974 64.887974) (end 147.202026 64.887974) (width 0.75) (layer B.Cu) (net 2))
 (segment (start 147.202026 64.887974) (end 150.368 61.722) (width 0.75) (layer B.Cu) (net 2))
 (segment (start 150.368 61.722) (end 152.146 61.722) (width 0.75) (layer B.Cu) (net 2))
 (segment (start 152.146 61.722) (end 152.654 61.722) (width 0.75) (layer B.Cu) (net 2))
 (segment (start 146.167974 64.887974) (end 146.167974 72.272026) (width 0.75) (layer B.Cu) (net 2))
 (segment (start 146.167974 72.272026) (end 145.288 73.152) (width 0.75) (layer B.Cu) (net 2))
 (segment (start 145.288 80.772) (end 144.78 81.28) (width 0.75) (layer B.Cu) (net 2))
 (segment (start 145.288 73.152) (end 145.288 80.772) (width 0.75) (layer B.Cu) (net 2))
 (segment (start 155.575 81.915) (end 153.7335 81.915) (width 0.75) (layer B.Cu) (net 2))
 (segment (start 157.48 83.82) (end 155.575 81.915) (width 0.75) (layer B.Cu) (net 2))
 (segment (start 153.7335 81.915) (end 150.368 85.2805) (width 0.75) (layer B.Cu) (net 2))
 (segment (start 150.368 85.2805) (end 150.368 86.36) (width 0.75) (layer B.Cu) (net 2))
 (segment (start 145.288 82.296) (end 145.288 80.772) (width 0.75) (layer B.Cu) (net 2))
 (segment (start 148.336 85.344) (end 145.288 82.296) (width 0.75) (layer B.Cu) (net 2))
 (segment (start 150.114 85.344) (end 148.336 85.344) (width 0.75) (layer B.Cu) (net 2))
 (segment (start 150.368 86.36) (end 150.368 85.598) (width 0.75) (layer B.Cu) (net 2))
 (segment (start 150.368 85.598) (end 150.114 85.344) (width 0.75) (layer B.Cu) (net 2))
 (segment (start 175.514 88.646) (end 175.514 86.106) (width 0.75) (layer B.Cu) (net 12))
 (segment (start 175.514 86.106) (end 179.705 81.915) (width 0.75) (layer B.Cu) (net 12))
 (segment (start 179.705 81.915) (end 179.705 73.025) (width 0.75) (layer B.Cu) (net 12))
 (segment (start 179.705 73.025) (end 177.8 71.12) (width 0.75) (layer B.Cu) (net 12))
 (segment (start 177.8 71.12) (end 175.26 71.12) (width 0.75) (layer B.Cu) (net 12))
 (segment (start 173.228 83.312) (end 173.228 83.82) (width 0.75) (layer B.Cu) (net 12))
 (segment (start 173.228 83.82) (end 175.514 86.106) (width 0.75) (layer B.Cu) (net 12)))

